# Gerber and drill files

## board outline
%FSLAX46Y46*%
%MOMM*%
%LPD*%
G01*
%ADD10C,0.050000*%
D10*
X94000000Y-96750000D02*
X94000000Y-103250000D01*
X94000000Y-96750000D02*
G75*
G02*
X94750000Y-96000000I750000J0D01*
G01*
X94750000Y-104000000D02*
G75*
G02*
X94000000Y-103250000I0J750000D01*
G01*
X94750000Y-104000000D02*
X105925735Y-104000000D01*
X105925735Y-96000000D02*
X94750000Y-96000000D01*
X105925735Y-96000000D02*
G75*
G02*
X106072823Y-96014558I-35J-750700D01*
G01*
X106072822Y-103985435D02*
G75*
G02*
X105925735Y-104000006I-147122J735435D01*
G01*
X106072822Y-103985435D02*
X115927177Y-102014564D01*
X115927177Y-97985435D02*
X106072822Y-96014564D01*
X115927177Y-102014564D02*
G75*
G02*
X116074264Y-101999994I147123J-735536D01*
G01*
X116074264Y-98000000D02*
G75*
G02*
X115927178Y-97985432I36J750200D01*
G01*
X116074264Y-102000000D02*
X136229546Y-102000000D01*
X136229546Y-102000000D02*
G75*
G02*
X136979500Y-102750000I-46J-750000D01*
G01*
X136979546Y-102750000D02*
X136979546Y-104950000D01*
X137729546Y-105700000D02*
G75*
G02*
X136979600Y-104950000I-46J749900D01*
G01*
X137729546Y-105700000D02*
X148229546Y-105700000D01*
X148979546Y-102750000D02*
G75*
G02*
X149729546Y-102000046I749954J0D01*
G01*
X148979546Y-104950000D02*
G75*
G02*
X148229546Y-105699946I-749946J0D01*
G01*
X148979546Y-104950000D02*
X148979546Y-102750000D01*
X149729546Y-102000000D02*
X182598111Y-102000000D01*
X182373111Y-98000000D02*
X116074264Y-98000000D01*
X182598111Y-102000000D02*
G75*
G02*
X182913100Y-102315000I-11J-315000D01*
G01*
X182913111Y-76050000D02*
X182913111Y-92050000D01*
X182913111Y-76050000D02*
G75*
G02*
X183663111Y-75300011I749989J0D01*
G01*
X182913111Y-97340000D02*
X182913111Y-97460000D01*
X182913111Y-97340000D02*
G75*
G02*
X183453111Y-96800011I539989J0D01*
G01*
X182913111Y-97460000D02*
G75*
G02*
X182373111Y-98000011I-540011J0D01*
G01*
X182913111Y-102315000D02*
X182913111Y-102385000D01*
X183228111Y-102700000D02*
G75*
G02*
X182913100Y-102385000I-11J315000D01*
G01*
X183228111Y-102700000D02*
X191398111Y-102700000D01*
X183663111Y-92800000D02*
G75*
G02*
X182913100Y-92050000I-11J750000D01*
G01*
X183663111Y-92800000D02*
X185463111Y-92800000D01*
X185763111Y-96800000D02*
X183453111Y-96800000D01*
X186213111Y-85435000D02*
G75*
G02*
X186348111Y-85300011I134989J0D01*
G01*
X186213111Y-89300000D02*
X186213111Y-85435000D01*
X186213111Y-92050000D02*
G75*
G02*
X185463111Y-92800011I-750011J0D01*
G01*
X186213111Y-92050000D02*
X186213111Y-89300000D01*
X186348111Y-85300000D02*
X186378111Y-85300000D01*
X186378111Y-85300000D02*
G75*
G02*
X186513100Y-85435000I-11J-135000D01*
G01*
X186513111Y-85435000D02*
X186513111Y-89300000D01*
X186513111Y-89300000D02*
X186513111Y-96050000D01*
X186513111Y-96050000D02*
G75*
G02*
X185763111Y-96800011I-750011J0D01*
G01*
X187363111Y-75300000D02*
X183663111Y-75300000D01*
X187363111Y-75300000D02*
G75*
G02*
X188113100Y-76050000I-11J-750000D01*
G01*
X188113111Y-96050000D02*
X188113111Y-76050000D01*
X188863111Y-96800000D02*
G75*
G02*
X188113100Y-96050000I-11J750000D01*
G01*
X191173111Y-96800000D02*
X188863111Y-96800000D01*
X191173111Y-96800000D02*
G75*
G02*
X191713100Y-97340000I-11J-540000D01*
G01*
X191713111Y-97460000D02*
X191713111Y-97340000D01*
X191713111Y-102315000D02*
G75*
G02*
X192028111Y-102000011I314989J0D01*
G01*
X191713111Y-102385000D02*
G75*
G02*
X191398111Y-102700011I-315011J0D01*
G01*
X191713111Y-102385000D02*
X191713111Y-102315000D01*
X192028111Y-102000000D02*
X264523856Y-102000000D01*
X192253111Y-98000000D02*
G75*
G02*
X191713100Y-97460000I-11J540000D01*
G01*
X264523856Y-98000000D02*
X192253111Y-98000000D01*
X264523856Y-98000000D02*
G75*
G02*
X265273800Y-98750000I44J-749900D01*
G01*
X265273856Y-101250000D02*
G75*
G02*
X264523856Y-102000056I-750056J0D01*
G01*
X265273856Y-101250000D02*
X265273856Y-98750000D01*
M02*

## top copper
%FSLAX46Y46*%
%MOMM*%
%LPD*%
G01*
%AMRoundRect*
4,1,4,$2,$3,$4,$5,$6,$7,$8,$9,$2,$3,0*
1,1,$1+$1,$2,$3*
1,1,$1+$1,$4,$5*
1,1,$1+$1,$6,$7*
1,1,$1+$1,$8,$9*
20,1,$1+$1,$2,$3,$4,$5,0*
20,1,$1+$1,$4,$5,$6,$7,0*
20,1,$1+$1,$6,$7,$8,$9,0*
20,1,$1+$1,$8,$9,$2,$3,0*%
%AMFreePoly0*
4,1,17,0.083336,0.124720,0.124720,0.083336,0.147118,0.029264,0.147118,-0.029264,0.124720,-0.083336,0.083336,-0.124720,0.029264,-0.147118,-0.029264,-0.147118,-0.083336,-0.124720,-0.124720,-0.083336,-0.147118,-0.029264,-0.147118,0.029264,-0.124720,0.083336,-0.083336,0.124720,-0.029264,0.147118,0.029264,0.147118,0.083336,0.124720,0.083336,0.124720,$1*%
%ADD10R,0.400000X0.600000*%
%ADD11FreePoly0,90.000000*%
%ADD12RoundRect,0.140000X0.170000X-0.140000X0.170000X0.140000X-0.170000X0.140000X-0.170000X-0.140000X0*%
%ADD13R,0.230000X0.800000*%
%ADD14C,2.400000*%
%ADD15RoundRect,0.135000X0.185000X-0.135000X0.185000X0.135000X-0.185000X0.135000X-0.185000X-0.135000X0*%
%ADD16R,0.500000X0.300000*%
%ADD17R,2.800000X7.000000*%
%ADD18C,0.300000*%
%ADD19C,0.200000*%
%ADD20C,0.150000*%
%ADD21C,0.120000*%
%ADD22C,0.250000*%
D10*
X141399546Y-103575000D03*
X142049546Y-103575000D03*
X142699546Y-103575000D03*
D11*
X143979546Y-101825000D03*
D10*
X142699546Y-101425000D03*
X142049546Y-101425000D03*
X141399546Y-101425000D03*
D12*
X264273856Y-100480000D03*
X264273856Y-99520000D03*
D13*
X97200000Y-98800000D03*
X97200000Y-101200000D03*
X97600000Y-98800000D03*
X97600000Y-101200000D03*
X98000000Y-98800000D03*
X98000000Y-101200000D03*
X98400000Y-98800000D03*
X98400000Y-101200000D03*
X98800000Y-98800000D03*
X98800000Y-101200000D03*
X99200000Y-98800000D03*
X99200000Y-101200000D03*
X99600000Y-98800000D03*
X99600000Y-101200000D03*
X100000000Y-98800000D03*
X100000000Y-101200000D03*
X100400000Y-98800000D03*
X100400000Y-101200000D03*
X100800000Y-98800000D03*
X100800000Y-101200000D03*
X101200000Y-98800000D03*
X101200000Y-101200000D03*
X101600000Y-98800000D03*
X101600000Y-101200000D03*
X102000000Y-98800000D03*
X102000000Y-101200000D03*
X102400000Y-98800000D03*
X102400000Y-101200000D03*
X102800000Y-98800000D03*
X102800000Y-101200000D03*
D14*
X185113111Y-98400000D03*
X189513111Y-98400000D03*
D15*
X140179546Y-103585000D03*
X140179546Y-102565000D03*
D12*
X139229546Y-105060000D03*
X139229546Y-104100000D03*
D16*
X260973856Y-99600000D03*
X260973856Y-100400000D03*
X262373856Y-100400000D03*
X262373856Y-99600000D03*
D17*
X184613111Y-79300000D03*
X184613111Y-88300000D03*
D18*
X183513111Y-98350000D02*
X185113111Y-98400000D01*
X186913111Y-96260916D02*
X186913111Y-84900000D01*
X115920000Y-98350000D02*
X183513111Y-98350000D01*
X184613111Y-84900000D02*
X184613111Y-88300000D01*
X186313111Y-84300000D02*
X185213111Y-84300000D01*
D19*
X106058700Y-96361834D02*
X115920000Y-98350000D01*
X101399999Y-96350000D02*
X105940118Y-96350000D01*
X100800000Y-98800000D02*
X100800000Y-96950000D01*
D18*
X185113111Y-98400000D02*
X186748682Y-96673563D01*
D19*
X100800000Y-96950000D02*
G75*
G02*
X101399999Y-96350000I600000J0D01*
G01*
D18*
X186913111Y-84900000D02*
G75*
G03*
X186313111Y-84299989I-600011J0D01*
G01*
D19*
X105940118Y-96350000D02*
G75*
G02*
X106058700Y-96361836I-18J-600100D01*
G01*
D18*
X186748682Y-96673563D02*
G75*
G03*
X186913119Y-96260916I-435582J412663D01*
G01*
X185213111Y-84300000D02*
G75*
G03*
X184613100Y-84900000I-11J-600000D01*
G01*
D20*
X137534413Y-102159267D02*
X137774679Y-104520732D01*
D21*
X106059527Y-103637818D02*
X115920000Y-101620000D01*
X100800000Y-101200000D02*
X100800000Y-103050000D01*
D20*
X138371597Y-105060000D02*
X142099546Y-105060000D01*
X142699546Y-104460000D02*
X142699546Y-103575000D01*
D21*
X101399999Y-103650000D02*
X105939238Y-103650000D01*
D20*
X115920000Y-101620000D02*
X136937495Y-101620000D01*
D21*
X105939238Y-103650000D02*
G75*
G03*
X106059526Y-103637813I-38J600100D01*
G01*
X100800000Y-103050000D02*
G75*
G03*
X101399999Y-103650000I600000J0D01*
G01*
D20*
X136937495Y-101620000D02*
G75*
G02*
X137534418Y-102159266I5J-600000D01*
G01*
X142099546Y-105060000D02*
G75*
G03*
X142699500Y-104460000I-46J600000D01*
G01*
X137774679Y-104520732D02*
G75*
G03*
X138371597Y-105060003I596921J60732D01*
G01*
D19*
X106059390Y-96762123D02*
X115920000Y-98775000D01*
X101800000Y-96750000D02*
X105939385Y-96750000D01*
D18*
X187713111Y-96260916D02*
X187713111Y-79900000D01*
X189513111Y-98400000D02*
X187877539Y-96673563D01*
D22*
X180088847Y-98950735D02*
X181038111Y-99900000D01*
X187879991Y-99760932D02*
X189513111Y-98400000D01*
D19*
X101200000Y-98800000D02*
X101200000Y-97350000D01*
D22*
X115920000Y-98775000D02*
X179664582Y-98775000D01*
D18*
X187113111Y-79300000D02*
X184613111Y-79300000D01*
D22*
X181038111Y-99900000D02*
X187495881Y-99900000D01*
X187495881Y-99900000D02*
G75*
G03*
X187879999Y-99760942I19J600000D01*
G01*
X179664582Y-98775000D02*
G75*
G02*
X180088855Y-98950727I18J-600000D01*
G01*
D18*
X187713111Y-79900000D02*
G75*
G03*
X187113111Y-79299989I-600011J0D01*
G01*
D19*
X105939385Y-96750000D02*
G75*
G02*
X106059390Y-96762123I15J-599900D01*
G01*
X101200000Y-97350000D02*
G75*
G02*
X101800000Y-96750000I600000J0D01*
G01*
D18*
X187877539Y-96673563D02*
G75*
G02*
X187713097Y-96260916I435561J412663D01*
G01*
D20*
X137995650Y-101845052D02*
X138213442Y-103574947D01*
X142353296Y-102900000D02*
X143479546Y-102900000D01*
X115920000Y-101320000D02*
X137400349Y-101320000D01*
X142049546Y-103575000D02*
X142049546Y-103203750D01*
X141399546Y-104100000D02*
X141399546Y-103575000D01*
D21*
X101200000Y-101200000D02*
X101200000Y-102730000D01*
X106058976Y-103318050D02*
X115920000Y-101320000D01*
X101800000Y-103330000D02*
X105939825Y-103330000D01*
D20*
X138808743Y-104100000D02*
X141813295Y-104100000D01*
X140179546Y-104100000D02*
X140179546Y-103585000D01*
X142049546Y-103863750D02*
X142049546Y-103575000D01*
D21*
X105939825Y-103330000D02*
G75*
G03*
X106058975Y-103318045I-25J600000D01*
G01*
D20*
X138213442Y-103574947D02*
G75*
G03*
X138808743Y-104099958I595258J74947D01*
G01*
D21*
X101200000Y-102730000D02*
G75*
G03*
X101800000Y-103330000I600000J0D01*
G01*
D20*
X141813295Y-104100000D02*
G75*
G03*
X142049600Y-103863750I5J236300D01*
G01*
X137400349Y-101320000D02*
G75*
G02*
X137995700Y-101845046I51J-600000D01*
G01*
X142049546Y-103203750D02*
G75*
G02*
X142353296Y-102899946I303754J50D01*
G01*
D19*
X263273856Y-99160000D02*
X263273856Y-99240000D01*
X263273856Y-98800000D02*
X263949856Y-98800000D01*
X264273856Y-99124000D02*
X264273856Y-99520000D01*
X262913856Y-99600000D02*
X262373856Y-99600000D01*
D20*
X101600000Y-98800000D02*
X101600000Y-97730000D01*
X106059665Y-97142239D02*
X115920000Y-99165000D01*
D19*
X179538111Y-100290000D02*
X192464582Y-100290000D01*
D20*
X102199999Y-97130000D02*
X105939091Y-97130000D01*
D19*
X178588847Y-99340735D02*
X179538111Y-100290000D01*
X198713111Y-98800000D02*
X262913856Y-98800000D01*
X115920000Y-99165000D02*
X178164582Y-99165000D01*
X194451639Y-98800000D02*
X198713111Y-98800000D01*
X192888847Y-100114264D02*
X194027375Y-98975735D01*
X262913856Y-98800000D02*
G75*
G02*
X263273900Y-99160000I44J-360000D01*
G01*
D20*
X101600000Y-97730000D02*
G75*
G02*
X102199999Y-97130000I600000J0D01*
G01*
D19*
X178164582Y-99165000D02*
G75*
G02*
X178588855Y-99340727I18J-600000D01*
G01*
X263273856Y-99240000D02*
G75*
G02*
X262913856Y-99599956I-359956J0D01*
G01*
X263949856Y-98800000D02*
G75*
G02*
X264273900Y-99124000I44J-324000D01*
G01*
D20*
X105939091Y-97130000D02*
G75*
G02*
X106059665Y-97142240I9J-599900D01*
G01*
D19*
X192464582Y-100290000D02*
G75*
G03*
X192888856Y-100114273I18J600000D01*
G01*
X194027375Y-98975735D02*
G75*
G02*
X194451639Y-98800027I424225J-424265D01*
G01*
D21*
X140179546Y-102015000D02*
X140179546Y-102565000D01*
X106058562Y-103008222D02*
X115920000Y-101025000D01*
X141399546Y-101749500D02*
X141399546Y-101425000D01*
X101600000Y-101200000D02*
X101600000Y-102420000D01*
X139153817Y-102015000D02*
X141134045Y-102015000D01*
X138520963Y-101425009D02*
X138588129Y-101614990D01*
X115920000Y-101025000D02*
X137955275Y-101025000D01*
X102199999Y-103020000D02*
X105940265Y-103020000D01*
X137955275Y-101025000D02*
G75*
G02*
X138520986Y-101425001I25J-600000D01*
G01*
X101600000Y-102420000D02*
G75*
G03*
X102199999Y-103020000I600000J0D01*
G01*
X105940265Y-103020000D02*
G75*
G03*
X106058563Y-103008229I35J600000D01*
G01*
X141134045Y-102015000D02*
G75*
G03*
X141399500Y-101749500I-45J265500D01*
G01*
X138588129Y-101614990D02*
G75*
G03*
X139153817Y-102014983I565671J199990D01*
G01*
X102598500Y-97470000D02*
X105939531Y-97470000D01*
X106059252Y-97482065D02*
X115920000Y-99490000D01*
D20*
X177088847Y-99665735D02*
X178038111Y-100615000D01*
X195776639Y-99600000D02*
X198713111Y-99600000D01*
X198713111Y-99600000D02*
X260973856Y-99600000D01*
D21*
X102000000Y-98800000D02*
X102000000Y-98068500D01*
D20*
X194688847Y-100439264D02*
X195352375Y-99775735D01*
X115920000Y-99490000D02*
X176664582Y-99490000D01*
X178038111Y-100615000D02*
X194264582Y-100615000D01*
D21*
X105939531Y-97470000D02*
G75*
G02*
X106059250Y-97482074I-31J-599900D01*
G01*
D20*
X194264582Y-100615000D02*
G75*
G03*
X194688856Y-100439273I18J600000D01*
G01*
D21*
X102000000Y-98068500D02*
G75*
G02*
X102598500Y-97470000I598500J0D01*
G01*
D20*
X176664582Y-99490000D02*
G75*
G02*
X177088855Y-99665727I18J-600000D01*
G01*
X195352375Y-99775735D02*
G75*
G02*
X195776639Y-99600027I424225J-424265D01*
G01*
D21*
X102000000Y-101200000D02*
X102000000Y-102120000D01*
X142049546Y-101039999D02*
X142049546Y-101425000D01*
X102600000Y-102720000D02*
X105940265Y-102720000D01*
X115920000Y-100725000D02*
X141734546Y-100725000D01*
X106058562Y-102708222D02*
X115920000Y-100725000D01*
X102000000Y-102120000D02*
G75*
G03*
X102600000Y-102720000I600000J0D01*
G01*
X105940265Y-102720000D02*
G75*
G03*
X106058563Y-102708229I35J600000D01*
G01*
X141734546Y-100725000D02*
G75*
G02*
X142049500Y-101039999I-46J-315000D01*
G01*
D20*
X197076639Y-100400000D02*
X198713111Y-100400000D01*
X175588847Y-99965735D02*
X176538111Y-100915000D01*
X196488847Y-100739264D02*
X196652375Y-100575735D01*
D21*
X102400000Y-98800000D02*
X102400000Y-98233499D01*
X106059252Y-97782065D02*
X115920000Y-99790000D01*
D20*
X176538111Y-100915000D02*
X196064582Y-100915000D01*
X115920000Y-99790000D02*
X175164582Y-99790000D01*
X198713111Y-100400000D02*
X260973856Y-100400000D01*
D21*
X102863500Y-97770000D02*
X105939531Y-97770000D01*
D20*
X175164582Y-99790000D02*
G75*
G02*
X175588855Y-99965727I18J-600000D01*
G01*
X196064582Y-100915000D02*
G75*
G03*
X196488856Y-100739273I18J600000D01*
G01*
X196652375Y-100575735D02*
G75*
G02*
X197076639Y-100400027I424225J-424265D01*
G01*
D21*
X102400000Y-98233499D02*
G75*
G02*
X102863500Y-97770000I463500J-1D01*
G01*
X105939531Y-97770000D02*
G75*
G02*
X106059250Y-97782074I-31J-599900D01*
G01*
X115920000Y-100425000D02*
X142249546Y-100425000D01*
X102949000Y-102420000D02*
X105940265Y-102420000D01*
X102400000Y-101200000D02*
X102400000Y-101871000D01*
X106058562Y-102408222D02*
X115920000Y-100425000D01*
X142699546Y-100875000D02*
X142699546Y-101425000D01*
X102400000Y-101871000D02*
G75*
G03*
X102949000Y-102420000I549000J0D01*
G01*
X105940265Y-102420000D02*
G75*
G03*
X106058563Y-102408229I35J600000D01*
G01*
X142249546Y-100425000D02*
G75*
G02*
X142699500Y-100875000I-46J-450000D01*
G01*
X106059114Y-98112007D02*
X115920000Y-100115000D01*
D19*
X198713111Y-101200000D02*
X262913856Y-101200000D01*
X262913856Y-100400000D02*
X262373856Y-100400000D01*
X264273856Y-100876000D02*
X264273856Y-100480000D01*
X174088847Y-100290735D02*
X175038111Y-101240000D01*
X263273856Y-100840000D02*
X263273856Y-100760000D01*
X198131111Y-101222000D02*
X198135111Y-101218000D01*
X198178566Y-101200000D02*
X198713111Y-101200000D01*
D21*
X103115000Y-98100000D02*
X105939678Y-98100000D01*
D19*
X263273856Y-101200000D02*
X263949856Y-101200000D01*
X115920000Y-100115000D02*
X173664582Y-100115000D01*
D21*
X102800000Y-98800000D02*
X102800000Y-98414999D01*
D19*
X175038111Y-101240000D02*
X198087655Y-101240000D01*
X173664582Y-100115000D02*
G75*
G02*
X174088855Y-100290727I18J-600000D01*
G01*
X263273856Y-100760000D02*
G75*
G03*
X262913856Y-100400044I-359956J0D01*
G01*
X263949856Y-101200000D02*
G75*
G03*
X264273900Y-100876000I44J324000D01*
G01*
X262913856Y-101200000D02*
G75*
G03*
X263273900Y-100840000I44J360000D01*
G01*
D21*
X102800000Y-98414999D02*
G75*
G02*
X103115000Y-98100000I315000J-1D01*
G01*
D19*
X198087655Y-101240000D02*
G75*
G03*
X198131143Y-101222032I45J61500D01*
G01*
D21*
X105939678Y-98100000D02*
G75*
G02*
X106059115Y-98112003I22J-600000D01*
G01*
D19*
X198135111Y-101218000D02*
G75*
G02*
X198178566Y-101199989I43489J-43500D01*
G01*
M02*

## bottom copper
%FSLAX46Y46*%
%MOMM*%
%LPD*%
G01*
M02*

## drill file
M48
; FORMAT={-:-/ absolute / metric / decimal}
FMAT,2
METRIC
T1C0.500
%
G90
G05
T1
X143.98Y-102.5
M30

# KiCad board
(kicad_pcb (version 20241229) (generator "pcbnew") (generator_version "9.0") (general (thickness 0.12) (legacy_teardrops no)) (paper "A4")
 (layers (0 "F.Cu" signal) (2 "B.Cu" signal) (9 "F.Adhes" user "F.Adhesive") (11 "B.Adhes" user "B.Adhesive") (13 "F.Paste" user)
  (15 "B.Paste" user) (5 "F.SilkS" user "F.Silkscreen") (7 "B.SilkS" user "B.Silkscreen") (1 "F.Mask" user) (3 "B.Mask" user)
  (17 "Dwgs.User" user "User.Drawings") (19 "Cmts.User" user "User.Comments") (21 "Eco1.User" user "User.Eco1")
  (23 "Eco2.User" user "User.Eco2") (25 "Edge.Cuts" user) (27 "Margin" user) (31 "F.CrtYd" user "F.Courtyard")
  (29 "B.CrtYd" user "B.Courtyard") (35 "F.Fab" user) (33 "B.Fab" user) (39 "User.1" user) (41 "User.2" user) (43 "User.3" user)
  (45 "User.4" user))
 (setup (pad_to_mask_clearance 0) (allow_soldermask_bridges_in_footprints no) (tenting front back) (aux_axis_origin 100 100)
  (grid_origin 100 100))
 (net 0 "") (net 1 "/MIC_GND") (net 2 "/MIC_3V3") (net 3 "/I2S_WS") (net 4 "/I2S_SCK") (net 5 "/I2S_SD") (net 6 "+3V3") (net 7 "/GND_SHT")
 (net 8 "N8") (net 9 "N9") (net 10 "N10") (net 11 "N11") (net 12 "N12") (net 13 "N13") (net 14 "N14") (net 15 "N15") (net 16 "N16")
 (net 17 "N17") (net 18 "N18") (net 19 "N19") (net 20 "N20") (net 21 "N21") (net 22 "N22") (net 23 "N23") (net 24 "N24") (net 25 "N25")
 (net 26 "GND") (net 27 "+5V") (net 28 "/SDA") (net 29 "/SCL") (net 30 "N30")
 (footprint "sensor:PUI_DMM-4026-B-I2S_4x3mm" (layer "F.Cu") (at 142.979546 102.5 90)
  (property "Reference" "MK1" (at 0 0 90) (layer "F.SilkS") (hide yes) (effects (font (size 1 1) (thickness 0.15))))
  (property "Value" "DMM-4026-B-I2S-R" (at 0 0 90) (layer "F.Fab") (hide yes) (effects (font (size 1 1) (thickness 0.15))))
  (pad "" np_thru_hole circle (at 0 1 90) (size 0.5 0.5) (drill 0.5) (layers "*.Mask"))
  (pad "1" smd rect (at -1.075 -1.58 90) (size 0.6 0.4) (layers "F.Cu" "F.Mask" "F.Paste") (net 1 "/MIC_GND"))
  (pad "2" smd rect (at -1.075 -0.93 90) (size 0.6 0.4) (layers "F.Cu" "F.Mask" "F.Paste") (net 1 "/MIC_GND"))
  (pad "3" smd rect (at -1.075 -0.28 90) (size 0.6 0.4) (layers "F.Cu" "F.Mask" "F.Paste") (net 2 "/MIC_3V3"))
  (pad "4" smd custom (at 0.675 1 90) (size 0.3 0.3) (layers "F.Cu" "F.Mask" "F.Paste") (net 1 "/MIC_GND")
   (options (clearance outline) (anchor circle)) (primitives))
  (pad "5" smd rect (at 1.075 -0.28 90) (size 0.6 0.4) (layers "F.Cu" "F.Mask" "F.Paste") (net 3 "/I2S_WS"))
  (pad "6" smd rect (at 1.075 -0.93 90) (size 0.6 0.4) (layers "F.Cu" "F.Mask" "F.Paste") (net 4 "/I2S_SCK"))
  (pad "7" smd rect (at 1.075 -1.58 90) (size 0.6 0.4) (layers "F.Cu" "F.Mask" "F.Paste") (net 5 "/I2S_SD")))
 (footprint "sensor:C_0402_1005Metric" (layer "F.Cu") (at 264.273856 100 90)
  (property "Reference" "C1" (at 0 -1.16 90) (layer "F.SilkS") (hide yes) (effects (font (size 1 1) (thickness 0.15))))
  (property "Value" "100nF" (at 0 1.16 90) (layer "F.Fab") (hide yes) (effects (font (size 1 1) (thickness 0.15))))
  (pad "1" smd roundrect (at -0.48 0 90) (size 0.56 0.62) (layers "F.Cu" "F.Mask" "F.Paste") (roundrect_rratio 0.25) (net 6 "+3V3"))
  (pad "2" smd roundrect (at 0.48 0 90) (size 0.56 0.62) (layers "F.Cu" "F.Mask" "F.Paste") (roundrect_rratio 0.25) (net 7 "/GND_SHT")))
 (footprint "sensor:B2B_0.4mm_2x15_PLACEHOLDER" (layer "F.Cu") (at 100 100)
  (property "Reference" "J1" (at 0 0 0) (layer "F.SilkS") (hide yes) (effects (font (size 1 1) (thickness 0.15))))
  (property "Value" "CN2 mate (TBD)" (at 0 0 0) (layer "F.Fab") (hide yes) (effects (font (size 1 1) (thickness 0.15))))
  (pad "1" smd rect (at -2.8 -1.2) (size 0.23 0.8) (layers "F.Cu" "F.Mask" "F.Paste") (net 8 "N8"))
  (pad "2" smd rect (at -2.8 1.2) (size 0.23 0.8) (layers "F.Cu" "F.Mask" "F.Paste") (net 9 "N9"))
  (pad "3" smd rect (at -2.4 -1.2) (size 0.23 0.8) (layers "F.Cu" "F.Mask" "F.Paste") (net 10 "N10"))
  (pad "4" smd rect (at -2.4 1.2) (size 0.23 0.8) (layers "F.Cu" "F.Mask" "F.Paste") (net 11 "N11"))
  (pad "5" smd rect (at -2 -1.2) (size 0.23 0.8) (layers "F.Cu" "F.Mask" "F.Paste") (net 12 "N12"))
  (pad "6" smd rect (at -2 1.2) (size 0.23 0.8) (layers "F.Cu" "F.Mask" "F.Paste") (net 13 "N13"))
  (pad "7" smd rect (at -1.6 -1.2) (size 0.23 0.8) (layers "F.Cu" "F.Mask" "F.Paste") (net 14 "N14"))
  (pad "8" smd rect (at -1.6 1.2) (size 0.23 0.8) (layers "F.Cu" "F.Mask" "F.Paste") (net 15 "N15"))
  (pad "9" smd rect (at -1.2 -1.2) (size 0.23 0.8) (layers "F.Cu" "F.Mask" "F.Paste") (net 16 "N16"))
  (pad "10" smd rect (at -1.2 1.2) (size 0.23 0.8) (layers "F.Cu" "F.Mask" "F.Paste") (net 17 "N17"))
  (pad "11" smd rect (at -0.8 -1.2) (size 0.23 0.8) (layers "F.Cu" "F.Mask" "F.Paste") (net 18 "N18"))
  (pad "12" smd rect (at -0.8 1.2) (size 0.23 0.8) (layers "F.Cu" "F.Mask" "F.Paste") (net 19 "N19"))
  (pad "13" smd rect (at -0.4 -1.2) (size 0.23 0.8) (layers "F.Cu" "F.Mask" "F.Paste") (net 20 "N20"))
  (pad "14" smd rect (at -0.4 1.2) (size 0.23 0.8) (layers "F.Cu" "F.Mask" "F.Paste") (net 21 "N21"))
  (pad "15" smd rect (at 0 -1.2) (size 0.23 0.8) (layers "F.Cu" "F.Mask" "F.Paste") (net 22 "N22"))
  (pad "16" smd rect (at 0 1.2) (size 0.23 0.8) (layers "F.Cu" "F.Mask" "F.Paste") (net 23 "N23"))
  (pad "17" smd rect (at 0.4 -1.2) (size 0.23 0.8) (layers "F.Cu" "F.Mask" "F.Paste") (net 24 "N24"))
  (pad "18" smd rect (at 0.4 1.2) (size 0.23 0.8) (layers "F.Cu" "F.Mask" "F.Paste") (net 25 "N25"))
  (pad "19" smd rect (at 0.8 -1.2) (size 0.23 0.8) (layers "F.Cu" "F.Mask" "F.Paste") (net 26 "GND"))
  (pad "20" smd rect (at 0.8 1.2) (size 0.23 0.8) (layers "F.Cu" "F.Mask" "F.Paste") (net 2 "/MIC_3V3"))
  (pad "21" smd rect (at 1.2 -1.2) (size 0.23 0.8) (layers "F.Cu" "F.Mask" "F.Paste") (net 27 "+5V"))
  (pad "22" smd rect (at 1.2 1.2) (size 0.23 0.8) (layers "F.Cu" "F.Mask" "F.Paste") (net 1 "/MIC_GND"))
  (pad "23" smd rect (at 1.6 -1.2) (size 0.23 0.8) (layers "F.Cu" "F.Mask" "F.Paste") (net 7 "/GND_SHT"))
  (pad "24" smd rect (at 1.6 1.2) (size 0.23 0.8) (layers "F.Cu" "F.Mask" "F.Paste") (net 5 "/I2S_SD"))
  (pad "25" smd rect (at 2 -1.2) (size 0.23 0.8) (layers "F.Cu" "F.Mask" "F.Paste") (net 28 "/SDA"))
  (pad "26" smd rect (at 2 1.2) (size 0.23 0.8) (layers "F.Cu" "F.Mask" "F.Paste") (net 4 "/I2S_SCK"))
  (pad "27" smd rect (at 2.4 -1.2) (size 0.23 0.8) (layers "F.Cu" "F.Mask" "F.Paste") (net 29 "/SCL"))
  (pad "28" smd rect (at 2.4 1.2) (size 0.23 0.8) (layers "F.Cu" "F.Mask" "F.Paste") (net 3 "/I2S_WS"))
  (pad "29" smd rect (at 2.8 -1.2) (size 0.23 0.8) (layers "F.Cu" "F.Mask" "F.Paste") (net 6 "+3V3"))
  (pad "30" smd rect (at 2.8 1.2) (size 0.23 0.8) (layers "F.Cu" "F.Mask" "F.Paste") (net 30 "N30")))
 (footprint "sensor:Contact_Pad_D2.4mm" (layer "F.Cu") (at 185.113111 98.4)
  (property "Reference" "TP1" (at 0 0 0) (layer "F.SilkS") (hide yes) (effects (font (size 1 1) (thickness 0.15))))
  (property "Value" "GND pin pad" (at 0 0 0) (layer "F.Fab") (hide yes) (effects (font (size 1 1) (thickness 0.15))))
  (pad "1" smd circle (at 0 0) (size 2.4 2.4) (layers "F.Cu" "F.Mask") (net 26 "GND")))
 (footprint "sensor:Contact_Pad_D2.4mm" (layer "F.Cu") (at 189.513111 98.4)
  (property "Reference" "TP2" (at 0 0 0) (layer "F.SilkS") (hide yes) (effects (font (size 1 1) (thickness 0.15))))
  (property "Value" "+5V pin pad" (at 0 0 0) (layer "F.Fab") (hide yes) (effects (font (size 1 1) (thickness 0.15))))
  (pad "1" smd circle (at 0 0) (size 2.4 2.4) (layers "F.Cu" "F.Mask") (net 27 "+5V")))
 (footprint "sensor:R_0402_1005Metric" (layer "F.Cu") (at 140.179546 103.075 90)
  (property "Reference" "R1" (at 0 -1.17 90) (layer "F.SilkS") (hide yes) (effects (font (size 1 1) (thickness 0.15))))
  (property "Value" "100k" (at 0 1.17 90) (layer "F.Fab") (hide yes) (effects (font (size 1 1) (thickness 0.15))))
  (pad "1" smd roundrect (at -0.51 0 90) (size 0.54 0.64) (layers "F.Cu" "F.Mask" "F.Paste") (roundrect_rratio 0.25) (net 1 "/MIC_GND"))
  (pad "2" smd roundrect (at 0.51 0 90) (size 0.54 0.64) (layers "F.Cu" "F.Mask" "F.Paste") (roundrect_rratio 0.25) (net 5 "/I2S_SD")))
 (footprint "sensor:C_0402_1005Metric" (layer "F.Cu") (at 139.229546 104.58 90)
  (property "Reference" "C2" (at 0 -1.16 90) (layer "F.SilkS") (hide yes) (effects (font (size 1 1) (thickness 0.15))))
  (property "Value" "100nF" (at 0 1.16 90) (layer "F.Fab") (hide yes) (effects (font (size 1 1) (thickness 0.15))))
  (pad "1" smd roundrect (at -0.48 0 90) (size 0.56 0.62) (layers "F.Cu" "F.Mask" "F.Paste") (roundrect_rratio 0.25) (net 2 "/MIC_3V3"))
  (pad "2" smd roundrect (at 0.48 0 90) (size 0.56 0.62) (layers "F.Cu" "F.Mask" "F.Paste") (roundrect_rratio 0.25) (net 1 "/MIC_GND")))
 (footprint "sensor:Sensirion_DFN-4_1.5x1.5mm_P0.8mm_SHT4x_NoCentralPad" (layer "F.Cu") (at 261.673856 100)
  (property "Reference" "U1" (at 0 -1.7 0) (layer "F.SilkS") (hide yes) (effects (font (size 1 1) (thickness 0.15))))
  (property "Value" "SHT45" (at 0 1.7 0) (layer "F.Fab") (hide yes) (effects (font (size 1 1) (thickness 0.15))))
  (pad "1" smd rect (at -0.7 -0.4) (size 0.5 0.3) (layers "F.Cu" "F.Mask" "F.Paste") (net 28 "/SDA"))
  (pad "2" smd rect (at -0.7 0.4) (size 0.5 0.3) (layers "F.Cu" "F.Mask" "F.Paste") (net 29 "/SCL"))
  (pad "3" smd rect (at 0.7 0.4) (size 0.5 0.3) (layers "F.Cu" "F.Mask" "F.Paste") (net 6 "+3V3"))
  (pad "4" smd rect (at 0.7 -0.4) (size 0.5 0.3) (layers "F.Cu" "F.Mask" "F.Paste") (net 7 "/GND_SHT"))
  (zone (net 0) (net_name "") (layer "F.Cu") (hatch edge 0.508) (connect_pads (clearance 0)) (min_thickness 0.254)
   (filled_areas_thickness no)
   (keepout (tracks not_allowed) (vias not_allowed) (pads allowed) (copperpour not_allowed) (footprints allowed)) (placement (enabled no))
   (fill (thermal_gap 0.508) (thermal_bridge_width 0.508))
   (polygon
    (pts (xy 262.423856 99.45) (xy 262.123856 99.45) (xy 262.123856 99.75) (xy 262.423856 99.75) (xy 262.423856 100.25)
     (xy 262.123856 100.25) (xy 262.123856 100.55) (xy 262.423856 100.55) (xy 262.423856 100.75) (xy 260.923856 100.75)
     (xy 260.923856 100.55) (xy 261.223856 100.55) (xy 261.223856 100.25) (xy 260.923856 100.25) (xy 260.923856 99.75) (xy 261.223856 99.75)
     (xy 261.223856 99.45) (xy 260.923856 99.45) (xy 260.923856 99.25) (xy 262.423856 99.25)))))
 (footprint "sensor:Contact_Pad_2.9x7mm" (layer "F.Cu") (at 184.613111 79.3)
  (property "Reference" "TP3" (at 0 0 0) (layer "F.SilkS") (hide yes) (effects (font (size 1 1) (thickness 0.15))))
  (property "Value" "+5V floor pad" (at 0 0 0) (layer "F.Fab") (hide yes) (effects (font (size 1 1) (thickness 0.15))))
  (pad "1" smd rect (at 0 0) (size 2.8 7) (layers "F.Cu" "F.Mask") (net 27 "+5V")))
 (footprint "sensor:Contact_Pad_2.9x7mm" (layer "F.Cu") (at 184.613111 88.3)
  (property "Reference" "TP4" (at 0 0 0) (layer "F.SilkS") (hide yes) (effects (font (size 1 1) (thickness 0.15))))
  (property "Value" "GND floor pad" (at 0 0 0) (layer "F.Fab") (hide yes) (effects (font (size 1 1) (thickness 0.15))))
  (pad "1" smd rect (at 0 0) (size 2.8 7) (layers "F.Cu" "F.Mask") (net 26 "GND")))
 (gr_line (start 94 96.75) (end 94 103.25) (stroke (width 0.05) (type default)) (layer "Edge.Cuts"))
 (gr_arc (start 94 96.75) (mid 94.21967 96.21967) (end 94.75 96) (stroke (width 0.05) (type default)) (layer "Edge.Cuts"))
 (gr_arc (start 94.75 104) (mid 94.21967 103.78033) (end 94 103.25) (stroke (width 0.05) (type default)) (layer "Edge.Cuts"))
 (gr_line (start 94.75 104) (end 105.925735 104) (stroke (width 0.05) (type default)) (layer "Edge.Cuts"))
 (gr_line (start 105.925735 96) (end 94.75 96) (stroke (width 0.05) (type default)) (layer "Edge.Cuts"))
 (gr_arc (start 105.925735 96) (mid 105.999638 96.003653) (end 106.072822 96.014564) (stroke (width 0.05) (type default))
  (layer "Edge.Cuts"))
 (gr_arc (start 106.072822 103.985435) (mid 105.999638 103.99635) (end 105.925735 104) (stroke (width 0.05) (type default))
  (layer "Edge.Cuts"))
 (gr_line (start 106.072822 103.985435) (end 115.927177 102.014564) (stroke (width 0.05) (type default)) (layer "Edge.Cuts"))
 (gr_line (start 115.927177 97.985435) (end 106.072822 96.014564) (stroke (width 0.05) (type default)) (layer "Edge.Cuts"))
 (gr_arc (start 115.927177 102.014564) (mid 116.000361 102.00365) (end 116.074264 102) (stroke (width 0.05) (type default))
  (layer "Edge.Cuts"))
 (gr_arc (start 116.074264 98) (mid 116.000361 97.996349) (end 115.927177 97.985435) (stroke (width 0.05) (type default))
  (layer "Edge.Cuts"))
 (gr_line (start 116.074264 102) (end 136.229546 102) (stroke (width 0.05) (type default)) (layer "Edge.Cuts"))
 (gr_arc (start 136.229546 102) (mid 136.759876 102.219669) (end 136.979546 102.75) (stroke (width 0.05) (type default)) (layer "Edge.Cuts"))
 (gr_line (start 136.979546 102.75) (end 136.979546 104.95) (stroke (width 0.05) (type default)) (layer "Edge.Cuts"))
 (gr_arc (start 137.729546 105.7) (mid 137.199186 105.480346) (end 136.979546 104.95) (stroke (width 0.05) (type default))
  (layer "Edge.Cuts"))
 (gr_line (start 137.729546 105.7) (end 148.229546 105.7) (stroke (width 0.05) (type default)) (layer "Edge.Cuts"))
 (gr_arc (start 148.979546 102.75) (mid 149.199216 102.219669) (end 149.729546 102) (stroke (width 0.05) (type default)) (layer "Edge.Cuts"))
 (gr_arc (start 148.979546 104.95) (mid 148.759879 105.480346) (end 148.229546 105.7) (stroke (width 0.05) (type default))
  (layer "Edge.Cuts"))
 (gr_line (start 148.979546 104.95) (end 148.979546 102.75) (stroke (width 0.05) (type default)) (layer "Edge.Cuts"))
 (gr_line (start 149.729546 102) (end 182.598111 102) (stroke (width 0.05) (type default)) (layer "Edge.Cuts"))
 (gr_line (start 182.373111 98) (end 116.074264 98) (stroke (width 0.05) (type default)) (layer "Edge.Cuts"))
 (gr_arc (start 182.598111 102) (mid 182.820849 102.092261) (end 182.913111 102.315) (stroke (width 0.05) (type default))
  (layer "Edge.Cuts"))
 (gr_line (start 182.913111 76.05) (end 182.913111 92.05) (stroke (width 0.05) (type default)) (layer "Edge.Cuts"))
 (gr_arc (start 182.913111 76.05) (mid 183.132782 75.519674) (end 183.663111 75.3) (stroke (width 0.05) (type default)) (layer "Edge.Cuts"))
 (gr_line (start 182.913111 97.34) (end 182.913111 97.46) (stroke (width 0.05) (type default)) (layer "Edge.Cuts"))
 (gr_arc (start 182.913111 97.34) (mid 183.071274 96.958166) (end 183.453111 96.8) (stroke (width 0.05) (type default)) (layer "Edge.Cuts"))
 (gr_arc (start 182.913111 97.46) (mid 182.754948 97.841837) (end 182.373111 98) (stroke (width 0.05) (type default)) (layer "Edge.Cuts"))
 (gr_line (start 182.913111 102.315) (end 182.913111 102.385) (stroke (width 0.05) (type default)) (layer "Edge.Cuts"))
 (gr_arc (start 183.228111 102.7) (mid 183.005365 102.607743) (end 182.913111 102.385) (stroke (width 0.05) (type default))
  (layer "Edge.Cuts"))
 (gr_line (start 183.228111 102.7) (end 191.398111 102.7) (stroke (width 0.05) (type default)) (layer "Edge.Cuts"))
 (gr_arc (start 183.663111 92.8) (mid 183.132774 92.580334) (end 182.913111 92.05) (stroke (width 0.05) (type default)) (layer "Edge.Cuts"))
 (gr_line (start 183.663111 92.8) (end 185.463111 92.8) (stroke (width 0.05) (type default)) (layer "Edge.Cuts"))
 (gr_line (start 185.763111 96.8) (end 183.453111 96.8) (stroke (width 0.05) (type default)) (layer "Edge.Cuts"))
 (gr_arc (start 186.213111 85.435) (mid 186.252651 85.33954) (end 186.348111 85.3) (stroke (width 0.05) (type default)) (layer "Edge.Cuts"))
 (gr_line (start 186.213111 89.3) (end 186.213111 85.435) (stroke (width 0.05) (type default)) (layer "Edge.Cuts"))
 (gr_arc (start 186.213111 92.05) (mid 185.993442 92.580334) (end 185.463111 92.8) (stroke (width 0.05) (type default)) (layer "Edge.Cuts"))
 (gr_line (start 186.213111 92.05) (end 186.213111 89.3) (stroke (width 0.05) (type default)) (layer "Edge.Cuts"))
 (gr_line (start 186.348111 85.3) (end 186.378111 85.3) (stroke (width 0.05) (type default)) (layer "Edge.Cuts"))
 (gr_arc (start 186.378111 85.3) (mid 186.47357 85.33954) (end 186.513111 85.435) (stroke (width 0.05) (type default)) (layer "Edge.Cuts"))
 (gr_line (start 186.513111 85.435) (end 186.513111 89.3) (stroke (width 0.05) (type default)) (layer "Edge.Cuts"))
 (gr_line (start 186.513111 89.3) (end 186.513111 96.05) (stroke (width 0.05) (type default)) (layer "Edge.Cuts"))
 (gr_arc (start 186.513111 96.05) (mid 186.293441 96.58033) (end 185.763111 96.8) (stroke (width 0.05) (type default)) (layer "Edge.Cuts"))
 (gr_line (start 187.363111 75.3) (end 183.663111 75.3) (stroke (width 0.05) (type default)) (layer "Edge.Cuts"))
 (gr_arc (start 187.363111 75.3) (mid 187.893434 75.519674) (end 188.113111 76.05) (stroke (width 0.05) (type default)) (layer "Edge.Cuts"))
 (gr_line (start 188.113111 96.05) (end 188.113111 76.05) (stroke (width 0.05) (type default)) (layer "Edge.Cuts"))
 (gr_arc (start 188.863111 96.8) (mid 188.332781 96.58033) (end 188.113111 96.05) (stroke (width 0.05) (type default)) (layer "Edge.Cuts"))
 (gr_line (start 191.173111 96.8) (end 188.863111 96.8) (stroke (width 0.05) (type default)) (layer "Edge.Cuts"))
 (gr_arc (start 191.173111 96.8) (mid 191.554942 96.958166) (end 191.713111 97.34) (stroke (width 0.05) (type default)) (layer "Edge.Cuts"))
 (gr_line (start 191.713111 97.46) (end 191.713111 97.34) (stroke (width 0.05) (type default)) (layer "Edge.Cuts"))
 (gr_arc (start 191.713111 102.315) (mid 191.805372 102.092261) (end 192.028111 102) (stroke (width 0.05) (type default))
  (layer "Edge.Cuts"))
 (gr_arc (start 191.713111 102.385) (mid 191.62085 102.607743) (end 191.398111 102.7) (stroke (width 0.05) (type default))
  (layer "Edge.Cuts"))
 (gr_line (start 191.713111 102.385) (end 191.713111 102.315) (stroke (width 0.05) (type default)) (layer "Edge.Cuts"))
 (gr_line (start 192.028111 102) (end 264.523856 102) (stroke (width 0.05) (type default)) (layer "Edge.Cuts"))
 (gr_arc (start 192.253111 98) (mid 191.871273 97.841837) (end 191.713111 97.46) (stroke (width 0.05) (type default)) (layer "Edge.Cuts"))
 (gr_line (start 264.523856 98) (end 192.253111 98) (stroke (width 0.05) (type default)) (layer "Edge.Cuts"))
 (gr_arc (start 264.523856 98) (mid 265.054215 98.219654) (end 265.273856 98.75) (stroke (width 0.05) (type default)) (layer "Edge.Cuts"))
 (gr_arc (start 265.273856 101.25) (mid 265.054183 101.780315) (end 264.523856 102) (stroke (width 0.05) (type default)) (layer "Edge.Cuts"))
 (gr_line (start 265.273856 101.25) (end 265.273856 98.75) (stroke (width 0.05) (type default)) (layer "Edge.Cuts"))
 (segment (start 183.513111 98.35) (end 185.113111 98.4) (width 0.3) (layer "F.Cu") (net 26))
 (segment (start 186.913111 96.260916) (end 186.913111 84.9) (width 0.3) (layer "F.Cu") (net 26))
 (segment (start 115.92 98.35) (end 183.513111 98.35) (width 0.3) (layer "F.Cu") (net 26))
 (segment (start 184.613111 84.9) (end 184.613111 88.3) (width 0.3) (layer "F.Cu") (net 26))
 (segment (start 186.313111 84.3) (end 185.213111 84.3) (width 0.3) (layer "F.Cu") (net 26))
 (segment (start 106.0587 96.361834) (end 115.92 98.35) (width 0.2) (layer "F.Cu") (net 26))
 (segment (start 101.399999 96.35) (end 105.940118 96.35) (width 0.2) (layer "F.Cu") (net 26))
 (segment (start 100.8 98.8) (end 100.8 96.95) (width 0.2) (layer "F.Cu") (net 26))
 (segment (start 185.113111 98.4) (end 186.748682 96.673563) (width 0.3) (layer "F.Cu") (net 26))
 (arc (start 100.8 96.95) (mid 100.975735 96.525735) (end 101.399999 96.35) (width 0.2) (layer "F.Cu") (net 26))
 (arc (start 186.913111 84.9) (mid 186.737375 84.475735) (end 186.313111 84.3) (width 0.3) (layer "F.Cu") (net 26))
 (arc (start 105.940118 96.35) (mid 105.999703 96.352966) (end 106.0587 96.361834) (width 0.2) (layer "F.Cu") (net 26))
 (arc (start 186.748682 96.673563) (mid 186.87049 96.483016) (end 186.913111 96.260916) (width 0.3) (layer "F.Cu") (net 26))
 (arc (start 185.213111 84.3) (mid 184.788846 84.475735) (end 184.613111 84.9) (width 0.3) (layer "F.Cu") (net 26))
 (segment (start 137.534413 102.159267) (end 137.774679 104.520732) (width 0.15) (layer "F.Cu") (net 2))
 (segment (start 106.059527 103.637818) (end 115.92 101.62) (width 0.12) (layer "F.Cu") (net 2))
 (segment (start 100.8 101.2) (end 100.8 103.05) (width 0.12) (layer "F.Cu") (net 2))
 (segment (start 138.371597 105.06) (end 142.099546 105.06) (width 0.15) (layer "F.Cu") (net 2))
 (segment (start 142.699546 104.46) (end 142.699546 103.575) (width 0.15) (layer "F.Cu") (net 2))
 (segment (start 101.399999 103.65) (end 105.939238 103.65) (width 0.12) (layer "F.Cu") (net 2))
 (segment (start 115.92 101.62) (end 136.937495 101.62) (width 0.15) (layer "F.Cu") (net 2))
 (arc (start 105.939238 103.65) (mid 105.99969 103.646946) (end 106.059527 103.637818) (width 0.12) (layer "F.Cu") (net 2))
 (arc (start 100.8 103.05) (mid 100.975735 103.474264) (end 101.399999 103.65) (width 0.12) (layer "F.Cu") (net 2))
 (arc (start 136.937495 101.62) (mid 137.339714 101.774781) (end 137.534413 102.159267) (width 0.15) (layer "F.Cu") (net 2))
 (arc (start 142.099546 105.06) (mid 142.52381 104.884264) (end 142.699546 104.46) (width 0.15) (layer "F.Cu") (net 2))
 (arc (start 137.774679 104.520732) (mid 137.969378 104.905218) (end 138.371597 105.06) (width 0.15) (layer "F.Cu") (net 2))
 (segment (start 106.05939 96.762123) (end 115.92 98.775) (width 0.2) (layer "F.Cu") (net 27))
 (segment (start 101.8 96.75) (end 105.939385 96.75) (width 0.2) (layer "F.Cu") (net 27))
 (segment (start 187.713111 96.260916) (end 187.713111 79.9) (width 0.3) (layer "F.Cu") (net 27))
 (segment (start 189.513111 98.4) (end 187.877539 96.673563) (width 0.3) (layer "F.Cu") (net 27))
 (segment (start 180.088847 98.950735) (end 181.038111 99.9) (width 0.25) (layer "F.Cu") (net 27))
 (segment (start 187.879991 99.760932) (end 189.513111 98.4) (width 0.25) (layer "F.Cu") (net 27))
 (segment (start 101.2 98.8) (end 101.2 97.35) (width 0.2) (layer "F.Cu") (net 27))
 (segment (start 115.92 98.775) (end 179.664582 98.775) (width 0.25) (layer "F.Cu") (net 27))
 (segment (start 187.113111 79.3) (end 184.613111 79.3) (width 0.3) (layer "F.Cu") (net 27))
 (segment (start 181.038111 99.9) (end 187.495881 99.9) (width 0.25) (layer "F.Cu") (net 27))
 (arc (start 187.495881 99.9) (mid 187.700136 99.864162) (end 187.879991 99.760932) (width 0.25) (layer "F.Cu") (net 27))
 (arc (start 179.664582 98.775) (mid 179.894193 98.820672) (end 180.088847 98.950735) (width 0.25) (layer "F.Cu") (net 27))
 (arc (start 187.713111 79.9) (mid 187.537375 79.475735) (end 187.113111 79.3) (width 0.3) (layer "F.Cu") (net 27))
 (arc (start 105.939385 96.75) (mid 105.999693 96.753038) (end 106.05939 96.762123) (width 0.2) (layer "F.Cu") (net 27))
 (arc (start 101.2 97.35) (mid 101.375735 96.925735) (end 101.8 96.75) (width 0.2) (layer "F.Cu") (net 27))
 (arc (start 187.877539 96.673563) (mid 187.755731 96.483016) (end 187.713111 96.260916) (width 0.3) (layer "F.Cu") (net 27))
 (segment (start 137.99565 101.845052) (end 138.213442 103.574947) (width 0.15) (layer "F.Cu") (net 1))
 (segment (start 142.353296 102.9) (end 143.479546 102.9) (width 0.15) (layer "F.Cu") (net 1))
 (segment (start 115.92 101.32) (end 137.400349 101.32) (width 0.15) (layer "F.Cu") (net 1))
 (segment (start 142.049546 103.575) (end 142.049546 103.20375) (width 0.15) (layer "F.Cu") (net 1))
 (segment (start 141.399546 104.1) (end 141.399546 103.575) (width 0.15) (layer "F.Cu") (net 1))
 (segment (start 101.2 101.2) (end 101.2 102.73) (width 0.12) (layer "F.Cu") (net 1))
 (segment (start 106.058976 103.31805) (end 115.92 101.32) (width 0.12) (layer "F.Cu") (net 1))
 (segment (start 101.8 103.33) (end 105.939825 103.33) (width 0.12) (layer "F.Cu") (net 1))
 (segment (start 138.808743 104.1) (end 141.813295 104.1) (width 0.15) (layer "F.Cu") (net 1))
 (segment (start 140.179546 104.1) (end 140.179546 103.585) (width 0.15) (layer "F.Cu") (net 1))
 (segment (start 142.049546 103.86375) (end 142.049546 103.575) (width 0.15) (layer "F.Cu") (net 1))
 (arc (start 105.939825 103.33) (mid 105.999699 103.327005) (end 106.058976 103.31805) (width 0.12) (layer "F.Cu") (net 1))
 (arc (start 138.213442 103.574947) (mid 138.411861 103.949982) (end 138.808743 104.1) (width 0.15) (layer "F.Cu") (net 1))
 (arc (start 101.2 102.73) (mid 101.375735 103.154264) (end 101.8 103.33) (width 0.12) (layer "F.Cu") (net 1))
 (arc (start 141.813295 104.1) (mid 141.980349 104.030803) (end 142.049546 103.86375) (width 0.15) (layer "F.Cu") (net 1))
 (arc (start 137.400349 101.32) (mid 137.797232 101.470017) (end 137.99565 101.845052) (width 0.15) (layer "F.Cu") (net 1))
 (arc (start 142.049546 103.20375) (mid 142.138512 102.988966) (end 142.353296 102.9) (width 0.15) (layer "F.Cu") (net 1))
 (segment (start 263.273856 99.16) (end 263.273856 99.24) (width 0.2) (layer "F.Cu") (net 7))
 (segment (start 263.273856 98.8) (end 263.949856 98.8) (width 0.2) (layer "F.Cu") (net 7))
 (segment (start 264.273856 99.124) (end 264.273856 99.52) (width 0.2) (layer "F.Cu") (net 7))
 (segment (start 262.913856 99.6) (end 262.373856 99.6) (width 0.2) (layer "F.Cu") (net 7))
 (segment (start 101.6 98.8) (end 101.6 97.73) (width 0.15) (layer "F.Cu") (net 7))
 (segment (start 106.059665 97.142239) (end 115.92 99.165) (width 0.15) (layer "F.Cu") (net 7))
 (segment (start 179.538111 100.29) (end 192.464582 100.29) (width 0.2) (layer "F.Cu") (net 7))
 (segment (start 102.199999 97.13) (end 105.939091 97.13) (width 0.15) (layer "F.Cu") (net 7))
 (segment (start 178.588847 99.340735) (end 179.538111 100.29) (width 0.2) (layer "F.Cu") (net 7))
 (segment (start 198.713111 98.8) (end 262.913856 98.8) (width 0.2) (layer "F.Cu") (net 7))
 (segment (start 115.92 99.165) (end 178.164582 99.165) (width 0.2) (layer "F.Cu") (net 7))
 (segment (start 194.451639 98.8) (end 198.713111 98.8) (width 0.2) (layer "F.Cu") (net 7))
 (segment (start 192.888847 100.114264) (end 194.027375 98.975735) (width 0.2) (layer "F.Cu") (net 7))
 (arc (start 262.913856 98.8) (mid 263.168414 98.905441) (end 263.273856 99.16) (width 0.2) (layer "F.Cu") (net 7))
 (arc (start 101.6 97.73) (mid 101.775735 97.305735) (end 102.199999 97.13) (width 0.15) (layer "F.Cu") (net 7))
 (arc (start 178.164582 99.165) (mid 178.394193 99.210672) (end 178.588847 99.340735) (width 0.2) (layer "F.Cu") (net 7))
 (arc (start 263.273856 99.24) (mid 263.168414 99.494558) (end 262.913856 99.6) (width 0.2) (layer "F.Cu") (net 7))
 (arc (start 263.949856 98.8) (mid 264.178958 98.894897) (end 264.273856 99.124) (width 0.2) (layer "F.Cu") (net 7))
 (arc (start 105.939091 97.13) (mid 105.999688 97.133067) (end 106.059665 97.142239) (width 0.15) (layer "F.Cu") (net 7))
 (arc (start 192.464582 100.29) (mid 192.694193 100.244327) (end 192.888847 100.114264) (width 0.2) (layer "F.Cu") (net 7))
 (arc (start 194.027375 98.975735) (mid 194.222029 98.845672) (end 194.451639 98.8) (width 0.2) (layer "F.Cu") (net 7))
 (segment (start 140.179546 102.015) (end 140.179546 102.565) (width 0.12) (layer "F.Cu") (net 5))
 (segment (start 106.058562 103.008222) (end 115.92 101.025) (width 0.12) (layer "F.Cu") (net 5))
 (segment (start 141.399546 101.7495) (end 141.399546 101.425) (width 0.12) (layer "F.Cu") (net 5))
 (segment (start 101.6 101.2) (end 101.6 102.42) (width 0.12) (layer "F.Cu") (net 5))
 (segment (start 139.153817 102.015) (end 141.134045 102.015) (width 0.12) (layer "F.Cu") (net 5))
 (segment (start 138.520963 101.425009) (end 138.588129 101.61499) (width 0.12) (layer "F.Cu") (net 5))
 (segment (start 115.92 101.025) (end 137.955275 101.025) (width 0.12) (layer "F.Cu") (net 5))
 (segment (start 102.199999 103.02) (end 105.940265 103.02) (width 0.12) (layer "F.Cu") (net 5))
 (arc (start 137.955275 101.025) (mid 138.301689 101.135104) (end 138.520963 101.425009) (width 0.12) (layer "F.Cu") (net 5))
 (arc (start 101.6 102.42) (mid 101.775735 102.844264) (end 102.199999 103.02) (width 0.12) (layer "F.Cu") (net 5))
 (arc (start 105.940265 103.02) (mid 105.999706 103.017048) (end 106.058562 103.008222) (width 0.12) (layer "F.Cu") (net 5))
 (arc (start 141.134045 102.015) (mid 141.321782 101.937236) (end 141.399546 101.7495) (width 0.12) (layer "F.Cu") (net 5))
 (arc (start 138.588129 101.61499) (mid 138.807403 101.904895) (end 139.153817 102.015) (width 0.12) (layer "F.Cu") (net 5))
 (segment (start 102.5985 97.47) (end 105.939531 97.47) (width 0.12) (layer "F.Cu") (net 28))
 (segment (start 106.059252 97.482065) (end 115.92 99.49) (width 0.12) (layer "F.Cu") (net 28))
 (segment (start 177.088847 99.665735) (end 178.038111 100.615) (width 0.15) (layer "F.Cu") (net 28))
 (segment (start 195.776639 99.6) (end 198.713111 99.6) (width 0.15) (layer "F.Cu") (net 28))
 (segment (start 198.713111 99.6) (end 260.973856 99.6) (width 0.15) (layer "F.Cu") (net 28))
 (segment (start 102 98.8) (end 102 98.0685) (width 0.12) (layer "F.Cu") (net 28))
 (segment (start 194.688847 100.439264) (end 195.352375 99.775735) (width 0.15) (layer "F.Cu") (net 28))
 (segment (start 115.92 99.49) (end 176.664582 99.49) (width 0.15) (layer "F.Cu") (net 28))
 (segment (start 178.038111 100.615) (end 194.264582 100.615) (width 0.15) (layer "F.Cu") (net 28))
 (arc (start 105.939531 97.47) (mid 105.999695 97.473023) (end 106.059252 97.482065) (width 0.12) (layer "F.Cu") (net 28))
 (arc (start 194.264582 100.615) (mid 194.494193 100.569327) (end 194.688847 100.439264) (width 0.15) (layer "F.Cu") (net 28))
 (arc (start 102 98.0685) (mid 102.175296 97.645296) (end 102.5985 97.47) (width 0.12) (layer "F.Cu") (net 28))
 (arc (start 176.664582 99.49) (mid 176.894193 99.535672) (end 177.088847 99.665735) (width 0.15) (layer "F.Cu") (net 28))
 (arc (start 195.352375 99.775735) (mid 195.547029 99.645672) (end 195.776639 99.6) (width 0.15) (layer "F.Cu") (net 28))
 (segment (start 102 101.2) (end 102 102.12) (width 0.12) (layer "F.Cu") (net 4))
 (segment (start 142.049546 101.039999) (end 142.049546 101.425) (width 0.12) (layer "F.Cu") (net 4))
 (segment (start 102.6 102.72) (end 105.940265 102.72) (width 0.12) (layer "F.Cu") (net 4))
 (segment (start 115.92 100.725) (end 141.734546 100.725) (width 0.12) (layer "F.Cu") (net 4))
 (segment (start 106.058562 102.708222) (end 115.92 100.725) (width 0.12) (layer "F.Cu") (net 4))
 (arc (start 102 102.12) (mid 102.175735 102.544264) (end 102.6 102.72) (width 0.12) (layer "F.Cu") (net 4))
 (arc (start 105.940265 102.72) (mid 105.999706 102.717048) (end 106.058562 102.708222) (width 0.12) (layer "F.Cu") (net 4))
 (arc (start 141.734546 100.725) (mid 141.957284 100.817261) (end 142.049546 101.039999) (width 0.12) (layer "F.Cu") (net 4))
 (segment (start 197.076639 100.4) (end 198.713111 100.4) (width 0.15) (layer "F.Cu") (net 29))
 (segment (start 175.588847 99.965735) (end 176.538111 100.915) (width 0.15) (layer "F.Cu") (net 29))
 (segment (start 196.488847 100.739264) (end 196.652375 100.575735) (width 0.15) (layer "F.Cu") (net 29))
 (segment (start 102.4 98.8) (end 102.4 98.233499) (width 0.12) (layer "F.Cu") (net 29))
 (segment (start 106.059252 97.782065) (end 115.92 99.79) (width 0.12) (layer "F.Cu") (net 29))
 (segment (start 176.538111 100.915) (end 196.064582 100.915) (width 0.15) (layer "F.Cu") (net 29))
 (segment (start 115.92 99.79) (end 175.164582 99.79) (width 0.15) (layer "F.Cu") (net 29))
 (segment (start 198.713111 100.4) (end 260.973856 100.4) (width 0.15) (layer "F.Cu") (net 29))
 (segment (start 102.8635 97.77) (end 105.939531 97.77) (width 0.12) (layer "F.Cu") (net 29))
 (arc (start 175.164582 99.79) (mid 175.394193 99.835672) (end 175.588847 99.965735) (width 0.15) (layer "F.Cu") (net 29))
 (arc (start 196.064582 100.915) (mid 196.294193 100.869327) (end 196.488847 100.739264) (width 0.15) (layer "F.Cu") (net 29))
 (arc (start 196.652375 100.575735) (mid 196.847029 100.445672) (end 197.076639 100.4) (width 0.15) (layer "F.Cu") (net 29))
 (arc (start 102.4 98.233499) (mid 102.535756 97.905756) (end 102.8635 97.77) (width 0.12) (layer "F.Cu") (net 29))
 (arc (start 105.939531 97.77) (mid 105.999695 97.773023) (end 106.059252 97.782065) (width 0.12) (layer "F.Cu") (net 29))
 (segment (start 115.92 100.425) (end 142.249546 100.425) (width 0.12) (layer "F.Cu") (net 3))
 (segment (start 102.949 102.42) (end 105.940265 102.42) (width 0.12) (layer "F.Cu") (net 3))
 (segment (start 102.4 101.2) (end 102.4 101.871) (width 0.12) (layer "F.Cu") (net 3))
 (segment (start 106.058562 102.408222) (end 115.92 100.425) (width 0.12) (layer "F.Cu") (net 3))
 (segment (start 142.699546 100.875) (end 142.699546 101.425) (width 0.12) (layer "F.Cu") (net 3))
 (arc (start 102.4 101.871) (mid 102.560798 102.259201) (end 102.949 102.42) (width 0.12) (layer "F.Cu") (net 3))
 (arc (start 105.940265 102.42) (mid 105.999706 102.417048) (end 106.058562 102.408222) (width 0.12) (layer "F.Cu") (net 3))
 (arc (start 142.249546 100.425) (mid 142.567744 100.556801) (end 142.699546 100.875) (width 0.12) (layer "F.Cu") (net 3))
 (segment (start 106.059114 98.112007) (end 115.92 100.115) (width 0.12) (layer "F.Cu") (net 6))
 (segment (start 198.713111 101.2) (end 262.913856 101.2) (width 0.2) (layer "F.Cu") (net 6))
 (segment (start 262.913856 100.4) (end 262.373856 100.4) (width 0.2) (layer "F.Cu") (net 6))
 (segment (start 264.273856 100.876) (end 264.273856 100.48) (width 0.2) (layer "F.Cu") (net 6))
 (segment (start 174.088847 100.290735) (end 175.038111 101.24) (width 0.2) (layer "F.Cu") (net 6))
 (segment (start 263.273856 100.84) (end 263.273856 100.76) (width 0.2) (layer "F.Cu") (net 6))
 (segment (start 198.131111 101.222) (end 198.135111 101.218) (width 0.2) (layer "F.Cu") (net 6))
 (segment (start 198.178566 101.2) (end 198.713111 101.2) (width 0.2) (layer "F.Cu") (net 6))
 (segment (start 103.115 98.1) (end 105.939678 98.1) (width 0.12) (layer "F.Cu") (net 6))
 (segment (start 263.273856 101.2) (end 263.949856 101.2) (width 0.2) (layer "F.Cu") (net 6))
 (segment (start 115.92 100.115) (end 173.664582 100.115) (width 0.2) (layer "F.Cu") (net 6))
 (segment (start 102.8 98.8) (end 102.8 98.414999) (width 0.12) (layer "F.Cu") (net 6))
 (segment (start 175.038111 101.24) (end 198.087655 101.24) (width 0.2) (layer "F.Cu") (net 6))
 (arc (start 173.664582 100.115) (mid 173.894193 100.160672) (end 174.088847 100.290735) (width 0.2) (layer "F.Cu") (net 6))
 (arc (start 263.273856 100.76) (mid 263.168414 100.505441) (end 262.913856 100.4) (width 0.2) (layer "F.Cu") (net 6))
 (arc (start 263.949856 101.2) (mid 264.178958 101.105102) (end 264.273856 100.876) (width 0.2) (layer "F.Cu") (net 6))
 (arc (start 262.913856 101.2) (mid 263.168414 101.094558) (end 263.273856 100.84) (width 0.2) (layer "F.Cu") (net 6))
 (arc (start 102.8 98.414999) (mid 102.892261 98.192261) (end 103.115 98.1) (width 0.12) (layer "F.Cu") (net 6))
 (arc (start 198.087655 101.24) (mid 198.111173 101.235321) (end 198.131111 101.222) (width 0.2) (layer "F.Cu") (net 6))
 (arc (start 105.939678 98.1) (mid 105.999697 98.103009) (end 106.059114 98.112007) (width 0.12) (layer "F.Cu") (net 6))
 (arc (start 198.135111 101.218) (mid 198.155048 101.204678) (end 198.178566 101.2) (width 0.2) (layer "F.Cu") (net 6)))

